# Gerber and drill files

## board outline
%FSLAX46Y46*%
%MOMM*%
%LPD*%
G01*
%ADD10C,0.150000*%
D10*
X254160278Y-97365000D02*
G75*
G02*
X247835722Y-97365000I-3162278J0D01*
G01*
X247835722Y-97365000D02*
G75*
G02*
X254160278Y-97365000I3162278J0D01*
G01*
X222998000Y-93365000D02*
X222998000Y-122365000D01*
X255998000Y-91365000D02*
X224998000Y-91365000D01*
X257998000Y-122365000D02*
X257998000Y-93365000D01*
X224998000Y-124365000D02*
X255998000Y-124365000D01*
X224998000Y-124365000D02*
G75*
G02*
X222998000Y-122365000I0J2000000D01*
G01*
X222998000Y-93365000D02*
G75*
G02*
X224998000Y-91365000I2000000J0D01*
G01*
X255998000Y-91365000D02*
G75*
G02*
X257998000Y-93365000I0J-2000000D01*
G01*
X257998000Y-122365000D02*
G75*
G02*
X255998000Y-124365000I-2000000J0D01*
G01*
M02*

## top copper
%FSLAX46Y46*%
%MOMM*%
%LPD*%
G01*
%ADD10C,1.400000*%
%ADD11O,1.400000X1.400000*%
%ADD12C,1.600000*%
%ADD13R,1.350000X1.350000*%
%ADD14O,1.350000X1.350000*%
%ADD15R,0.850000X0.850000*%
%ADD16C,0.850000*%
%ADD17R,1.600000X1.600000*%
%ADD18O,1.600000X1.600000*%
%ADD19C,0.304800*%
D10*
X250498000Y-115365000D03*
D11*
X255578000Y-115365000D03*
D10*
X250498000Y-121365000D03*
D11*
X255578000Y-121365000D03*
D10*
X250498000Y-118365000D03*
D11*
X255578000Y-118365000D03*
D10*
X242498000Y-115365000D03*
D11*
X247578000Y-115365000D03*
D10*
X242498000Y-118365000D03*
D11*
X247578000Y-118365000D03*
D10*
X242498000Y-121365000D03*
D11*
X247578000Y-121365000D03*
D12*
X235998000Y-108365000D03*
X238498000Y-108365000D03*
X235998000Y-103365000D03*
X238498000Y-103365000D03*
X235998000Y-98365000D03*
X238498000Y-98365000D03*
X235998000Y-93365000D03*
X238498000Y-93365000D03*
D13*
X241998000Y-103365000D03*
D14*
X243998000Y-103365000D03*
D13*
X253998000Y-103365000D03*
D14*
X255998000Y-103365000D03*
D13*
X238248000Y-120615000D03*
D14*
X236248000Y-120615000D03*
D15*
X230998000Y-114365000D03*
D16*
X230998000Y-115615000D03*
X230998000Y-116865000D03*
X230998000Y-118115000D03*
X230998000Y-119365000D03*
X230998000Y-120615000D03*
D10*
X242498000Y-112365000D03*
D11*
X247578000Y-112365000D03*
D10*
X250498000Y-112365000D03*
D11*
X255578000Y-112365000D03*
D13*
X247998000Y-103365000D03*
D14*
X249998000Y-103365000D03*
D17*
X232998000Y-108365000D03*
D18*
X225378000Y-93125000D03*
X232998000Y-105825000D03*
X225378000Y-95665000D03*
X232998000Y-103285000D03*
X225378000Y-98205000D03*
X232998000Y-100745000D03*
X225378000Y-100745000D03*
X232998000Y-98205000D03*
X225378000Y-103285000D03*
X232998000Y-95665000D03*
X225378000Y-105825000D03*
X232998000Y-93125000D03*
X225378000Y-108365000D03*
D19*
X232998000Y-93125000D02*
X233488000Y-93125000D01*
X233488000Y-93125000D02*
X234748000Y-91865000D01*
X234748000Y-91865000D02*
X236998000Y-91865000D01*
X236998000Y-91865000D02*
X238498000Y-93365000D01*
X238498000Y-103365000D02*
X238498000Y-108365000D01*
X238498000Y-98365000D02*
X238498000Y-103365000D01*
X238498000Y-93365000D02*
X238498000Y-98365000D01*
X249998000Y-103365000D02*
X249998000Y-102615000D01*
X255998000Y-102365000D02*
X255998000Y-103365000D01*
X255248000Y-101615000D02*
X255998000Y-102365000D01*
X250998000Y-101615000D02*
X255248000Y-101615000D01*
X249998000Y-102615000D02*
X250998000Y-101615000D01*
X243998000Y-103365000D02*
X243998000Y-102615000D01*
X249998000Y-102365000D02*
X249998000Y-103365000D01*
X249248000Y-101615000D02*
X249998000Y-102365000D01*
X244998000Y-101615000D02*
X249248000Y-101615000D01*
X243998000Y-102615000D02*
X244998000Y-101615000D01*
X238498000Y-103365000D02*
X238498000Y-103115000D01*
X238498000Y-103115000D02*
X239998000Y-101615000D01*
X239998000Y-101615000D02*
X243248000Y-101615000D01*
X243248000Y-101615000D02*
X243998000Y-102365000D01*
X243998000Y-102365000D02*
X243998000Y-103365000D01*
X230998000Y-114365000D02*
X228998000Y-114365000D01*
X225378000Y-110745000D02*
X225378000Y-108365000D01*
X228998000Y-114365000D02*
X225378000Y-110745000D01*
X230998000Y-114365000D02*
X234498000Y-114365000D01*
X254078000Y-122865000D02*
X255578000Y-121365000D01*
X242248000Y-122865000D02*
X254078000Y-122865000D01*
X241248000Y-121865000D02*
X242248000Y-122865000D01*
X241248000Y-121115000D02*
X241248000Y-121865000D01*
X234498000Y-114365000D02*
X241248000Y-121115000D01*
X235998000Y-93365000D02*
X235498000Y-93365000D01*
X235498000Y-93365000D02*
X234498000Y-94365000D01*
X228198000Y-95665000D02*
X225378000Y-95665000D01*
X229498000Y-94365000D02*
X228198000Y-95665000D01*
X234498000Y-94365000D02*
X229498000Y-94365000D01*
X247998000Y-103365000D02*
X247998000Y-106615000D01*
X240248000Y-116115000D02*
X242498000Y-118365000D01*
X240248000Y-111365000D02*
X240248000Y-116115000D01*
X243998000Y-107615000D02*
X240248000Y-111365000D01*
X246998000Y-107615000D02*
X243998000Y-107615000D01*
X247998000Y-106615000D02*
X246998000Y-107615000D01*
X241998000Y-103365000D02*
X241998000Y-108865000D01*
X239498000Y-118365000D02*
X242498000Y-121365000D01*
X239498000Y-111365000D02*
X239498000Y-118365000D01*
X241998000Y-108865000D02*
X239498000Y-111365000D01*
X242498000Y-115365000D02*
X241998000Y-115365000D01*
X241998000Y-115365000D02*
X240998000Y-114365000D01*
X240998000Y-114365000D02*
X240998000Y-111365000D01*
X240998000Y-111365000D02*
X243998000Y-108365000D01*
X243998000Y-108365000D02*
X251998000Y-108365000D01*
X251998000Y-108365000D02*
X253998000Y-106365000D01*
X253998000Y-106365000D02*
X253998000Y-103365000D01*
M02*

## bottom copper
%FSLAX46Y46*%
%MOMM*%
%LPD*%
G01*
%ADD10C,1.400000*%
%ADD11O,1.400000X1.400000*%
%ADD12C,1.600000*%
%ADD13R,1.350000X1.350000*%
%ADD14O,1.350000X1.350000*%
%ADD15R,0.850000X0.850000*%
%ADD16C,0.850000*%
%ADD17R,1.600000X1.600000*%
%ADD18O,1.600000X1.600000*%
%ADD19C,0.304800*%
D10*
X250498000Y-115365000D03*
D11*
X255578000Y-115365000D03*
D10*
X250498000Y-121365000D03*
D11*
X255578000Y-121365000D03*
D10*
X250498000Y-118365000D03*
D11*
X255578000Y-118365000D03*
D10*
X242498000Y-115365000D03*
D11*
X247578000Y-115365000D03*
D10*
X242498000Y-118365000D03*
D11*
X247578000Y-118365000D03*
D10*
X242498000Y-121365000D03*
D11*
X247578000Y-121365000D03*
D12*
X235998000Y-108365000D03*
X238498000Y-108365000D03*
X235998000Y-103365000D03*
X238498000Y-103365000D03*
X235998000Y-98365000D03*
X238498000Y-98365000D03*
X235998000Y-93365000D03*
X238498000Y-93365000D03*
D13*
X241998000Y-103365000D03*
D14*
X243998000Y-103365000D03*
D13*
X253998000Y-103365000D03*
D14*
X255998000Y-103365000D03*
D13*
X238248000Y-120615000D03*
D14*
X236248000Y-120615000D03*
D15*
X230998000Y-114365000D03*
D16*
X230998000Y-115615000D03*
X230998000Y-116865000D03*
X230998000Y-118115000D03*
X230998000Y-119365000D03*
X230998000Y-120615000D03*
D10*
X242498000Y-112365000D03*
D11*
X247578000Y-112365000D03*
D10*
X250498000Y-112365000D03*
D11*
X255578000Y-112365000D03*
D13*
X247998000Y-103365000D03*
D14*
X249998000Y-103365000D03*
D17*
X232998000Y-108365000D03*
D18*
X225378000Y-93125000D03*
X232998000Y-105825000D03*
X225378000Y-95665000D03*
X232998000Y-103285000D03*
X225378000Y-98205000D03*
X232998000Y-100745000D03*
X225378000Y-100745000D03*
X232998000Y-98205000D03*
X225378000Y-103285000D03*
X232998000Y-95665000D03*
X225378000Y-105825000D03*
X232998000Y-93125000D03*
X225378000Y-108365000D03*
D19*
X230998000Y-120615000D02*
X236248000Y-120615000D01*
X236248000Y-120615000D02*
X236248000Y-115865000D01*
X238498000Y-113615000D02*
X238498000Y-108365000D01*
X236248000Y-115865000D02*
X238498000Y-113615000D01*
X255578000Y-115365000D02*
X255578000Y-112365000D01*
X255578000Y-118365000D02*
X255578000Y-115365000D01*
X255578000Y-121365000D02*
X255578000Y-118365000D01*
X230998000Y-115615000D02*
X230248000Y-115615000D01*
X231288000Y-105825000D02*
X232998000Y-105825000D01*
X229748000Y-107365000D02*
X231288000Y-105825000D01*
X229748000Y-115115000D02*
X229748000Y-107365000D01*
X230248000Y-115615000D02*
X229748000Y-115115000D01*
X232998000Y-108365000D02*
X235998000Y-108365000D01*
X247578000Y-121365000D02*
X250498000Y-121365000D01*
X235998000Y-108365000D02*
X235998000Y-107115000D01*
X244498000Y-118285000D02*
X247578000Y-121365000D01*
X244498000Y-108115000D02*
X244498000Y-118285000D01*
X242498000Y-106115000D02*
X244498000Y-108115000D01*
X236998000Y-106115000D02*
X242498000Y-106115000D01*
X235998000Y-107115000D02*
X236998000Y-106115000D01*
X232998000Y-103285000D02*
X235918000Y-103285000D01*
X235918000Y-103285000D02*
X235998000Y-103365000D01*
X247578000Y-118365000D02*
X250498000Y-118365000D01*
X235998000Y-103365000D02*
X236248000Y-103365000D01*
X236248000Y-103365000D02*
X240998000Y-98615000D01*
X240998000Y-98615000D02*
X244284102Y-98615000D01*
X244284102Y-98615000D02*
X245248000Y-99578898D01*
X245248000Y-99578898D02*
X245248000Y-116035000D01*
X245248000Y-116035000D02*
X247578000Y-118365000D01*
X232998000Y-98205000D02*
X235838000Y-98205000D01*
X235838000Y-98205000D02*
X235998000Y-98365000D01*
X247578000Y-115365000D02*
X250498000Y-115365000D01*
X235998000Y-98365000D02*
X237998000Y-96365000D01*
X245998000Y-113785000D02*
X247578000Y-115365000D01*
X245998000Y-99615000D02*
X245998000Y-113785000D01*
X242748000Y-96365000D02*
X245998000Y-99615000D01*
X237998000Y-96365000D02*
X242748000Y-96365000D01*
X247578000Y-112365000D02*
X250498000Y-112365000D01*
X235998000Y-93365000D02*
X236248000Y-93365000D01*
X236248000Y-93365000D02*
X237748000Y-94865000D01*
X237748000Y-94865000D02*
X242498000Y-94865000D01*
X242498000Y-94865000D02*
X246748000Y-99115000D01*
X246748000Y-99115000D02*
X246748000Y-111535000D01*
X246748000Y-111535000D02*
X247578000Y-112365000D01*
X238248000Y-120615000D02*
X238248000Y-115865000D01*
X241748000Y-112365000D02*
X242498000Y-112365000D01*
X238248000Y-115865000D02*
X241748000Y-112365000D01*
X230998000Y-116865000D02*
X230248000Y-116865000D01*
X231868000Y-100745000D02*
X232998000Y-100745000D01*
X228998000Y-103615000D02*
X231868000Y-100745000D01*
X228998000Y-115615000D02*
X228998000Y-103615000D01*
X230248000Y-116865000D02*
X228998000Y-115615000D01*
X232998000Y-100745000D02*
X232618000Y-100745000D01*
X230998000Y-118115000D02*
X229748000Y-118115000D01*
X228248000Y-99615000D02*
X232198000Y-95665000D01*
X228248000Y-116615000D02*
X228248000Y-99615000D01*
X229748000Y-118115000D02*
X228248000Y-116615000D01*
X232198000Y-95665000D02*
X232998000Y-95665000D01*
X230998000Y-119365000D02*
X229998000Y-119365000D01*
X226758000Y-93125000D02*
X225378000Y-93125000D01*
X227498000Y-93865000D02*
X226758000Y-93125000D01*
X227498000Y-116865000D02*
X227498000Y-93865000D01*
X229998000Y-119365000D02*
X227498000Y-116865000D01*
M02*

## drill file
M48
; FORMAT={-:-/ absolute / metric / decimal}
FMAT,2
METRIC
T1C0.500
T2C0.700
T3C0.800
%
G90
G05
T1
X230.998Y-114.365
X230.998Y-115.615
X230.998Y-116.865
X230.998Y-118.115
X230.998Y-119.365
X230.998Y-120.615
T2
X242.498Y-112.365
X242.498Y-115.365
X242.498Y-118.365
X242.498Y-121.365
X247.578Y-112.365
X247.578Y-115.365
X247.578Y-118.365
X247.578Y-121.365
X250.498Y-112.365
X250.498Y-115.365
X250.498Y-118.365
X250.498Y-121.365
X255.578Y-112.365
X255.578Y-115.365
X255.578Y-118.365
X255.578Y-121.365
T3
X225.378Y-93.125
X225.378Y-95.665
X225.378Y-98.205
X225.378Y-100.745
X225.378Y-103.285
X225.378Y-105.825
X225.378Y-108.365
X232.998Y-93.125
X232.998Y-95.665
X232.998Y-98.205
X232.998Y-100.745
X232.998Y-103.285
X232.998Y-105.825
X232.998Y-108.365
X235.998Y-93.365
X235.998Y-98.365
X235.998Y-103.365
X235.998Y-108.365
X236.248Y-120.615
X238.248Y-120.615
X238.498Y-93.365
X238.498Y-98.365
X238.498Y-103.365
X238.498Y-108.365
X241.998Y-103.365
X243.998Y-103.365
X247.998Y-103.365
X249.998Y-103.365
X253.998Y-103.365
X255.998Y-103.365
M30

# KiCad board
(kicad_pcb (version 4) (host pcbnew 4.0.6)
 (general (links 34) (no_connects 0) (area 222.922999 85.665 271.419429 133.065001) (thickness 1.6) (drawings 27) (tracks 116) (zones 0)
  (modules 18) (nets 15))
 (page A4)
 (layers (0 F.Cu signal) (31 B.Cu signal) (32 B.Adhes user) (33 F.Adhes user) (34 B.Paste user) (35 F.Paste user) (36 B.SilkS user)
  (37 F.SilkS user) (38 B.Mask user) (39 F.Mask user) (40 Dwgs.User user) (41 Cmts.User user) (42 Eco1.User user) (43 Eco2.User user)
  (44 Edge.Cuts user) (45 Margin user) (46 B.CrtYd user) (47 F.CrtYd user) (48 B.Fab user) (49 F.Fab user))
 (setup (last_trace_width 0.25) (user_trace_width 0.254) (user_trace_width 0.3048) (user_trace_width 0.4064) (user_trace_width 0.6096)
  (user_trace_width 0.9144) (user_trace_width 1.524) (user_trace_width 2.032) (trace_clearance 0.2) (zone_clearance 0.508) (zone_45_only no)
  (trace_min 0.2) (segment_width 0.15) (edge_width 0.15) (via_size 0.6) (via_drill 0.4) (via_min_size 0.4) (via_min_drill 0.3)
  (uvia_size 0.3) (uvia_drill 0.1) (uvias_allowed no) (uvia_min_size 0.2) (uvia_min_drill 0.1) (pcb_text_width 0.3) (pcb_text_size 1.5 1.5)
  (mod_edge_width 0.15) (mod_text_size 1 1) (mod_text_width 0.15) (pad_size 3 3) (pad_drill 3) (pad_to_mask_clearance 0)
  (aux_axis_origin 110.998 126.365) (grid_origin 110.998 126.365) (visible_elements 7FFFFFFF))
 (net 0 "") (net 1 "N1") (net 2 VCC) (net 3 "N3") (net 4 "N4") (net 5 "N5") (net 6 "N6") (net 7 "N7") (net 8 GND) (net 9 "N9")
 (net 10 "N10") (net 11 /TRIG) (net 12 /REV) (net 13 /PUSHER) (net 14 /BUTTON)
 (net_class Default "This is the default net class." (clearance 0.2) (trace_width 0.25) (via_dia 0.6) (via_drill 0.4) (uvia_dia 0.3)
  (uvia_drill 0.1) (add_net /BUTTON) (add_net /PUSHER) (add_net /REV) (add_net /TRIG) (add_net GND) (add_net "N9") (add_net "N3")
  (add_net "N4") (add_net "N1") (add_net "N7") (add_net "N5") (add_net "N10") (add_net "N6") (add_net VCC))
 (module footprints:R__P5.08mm (layer F.Cu) (at 252.998 115.365)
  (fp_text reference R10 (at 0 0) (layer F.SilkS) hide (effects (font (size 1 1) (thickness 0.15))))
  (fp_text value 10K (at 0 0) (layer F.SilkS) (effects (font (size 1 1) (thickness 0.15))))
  (pad 1 thru_hole circle (at -2.5 0) (size 1.4 1.4) (drill 0.7) (layers *.Cu *.Mask) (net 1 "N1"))
  (pad 2 thru_hole oval (at 2.58 0) (size 1.4 1.4) (drill 0.7) (layers *.Cu *.Mask) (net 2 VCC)))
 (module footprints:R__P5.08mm (layer F.Cu) (at 252.998 121.365)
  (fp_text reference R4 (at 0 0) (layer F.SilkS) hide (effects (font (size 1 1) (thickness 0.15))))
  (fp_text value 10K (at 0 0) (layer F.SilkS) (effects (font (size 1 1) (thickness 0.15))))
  (pad 1 thru_hole circle (at -2.5 0) (size 1.4 1.4) (drill 0.7) (layers *.Cu *.Mask) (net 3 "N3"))
  (pad 2 thru_hole oval (at 2.58 0) (size 1.4 1.4) (drill 0.7) (layers *.Cu *.Mask) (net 2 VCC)))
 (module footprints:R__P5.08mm (layer F.Cu) (at 252.998 118.365)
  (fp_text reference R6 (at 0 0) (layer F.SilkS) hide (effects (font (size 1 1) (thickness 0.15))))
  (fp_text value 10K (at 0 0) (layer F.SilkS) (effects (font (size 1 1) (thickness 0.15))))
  (pad 1 thru_hole circle (at -2.5 0) (size 1.4 1.4) (drill 0.7) (layers *.Cu *.Mask) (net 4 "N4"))
  (pad 2 thru_hole oval (at 2.58 0) (size 1.4 1.4) (drill 0.7) (layers *.Cu *.Mask) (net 2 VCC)))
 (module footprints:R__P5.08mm (layer F.Cu) (at 244.998 115.365)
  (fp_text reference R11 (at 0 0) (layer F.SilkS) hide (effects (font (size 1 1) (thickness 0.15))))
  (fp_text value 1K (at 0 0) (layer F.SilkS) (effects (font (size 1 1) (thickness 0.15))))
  (pad 1 thru_hole circle (at -2.5 0) (size 1.4 1.4) (drill 0.7) (layers *.Cu *.Mask) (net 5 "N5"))
  (pad 2 thru_hole oval (at 2.58 0) (size 1.4 1.4) (drill 0.7) (layers *.Cu *.Mask) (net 1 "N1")))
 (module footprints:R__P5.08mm (layer F.Cu) (at 244.998 118.365)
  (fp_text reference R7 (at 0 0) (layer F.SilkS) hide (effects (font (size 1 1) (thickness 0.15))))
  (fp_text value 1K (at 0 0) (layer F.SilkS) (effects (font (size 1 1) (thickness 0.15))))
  (pad 1 thru_hole circle (at -2.5 0) (size 1.4 1.4) (drill 0.7) (layers *.Cu *.Mask) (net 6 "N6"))
  (pad 2 thru_hole oval (at 2.58 0) (size 1.4 1.4) (drill 0.7) (layers *.Cu *.Mask) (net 4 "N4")))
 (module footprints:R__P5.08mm (layer F.Cu) (at 244.998 121.365)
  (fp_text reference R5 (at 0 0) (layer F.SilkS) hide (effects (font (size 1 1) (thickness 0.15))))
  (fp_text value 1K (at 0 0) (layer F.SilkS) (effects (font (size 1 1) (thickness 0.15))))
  (pad 1 thru_hole circle (at -2.5 0) (size 1.4 1.4) (drill 0.7) (layers *.Cu *.Mask) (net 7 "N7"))
  (pad 2 thru_hole oval (at 2.58 0) (size 1.4 1.4) (drill 0.7) (layers *.Cu *.Mask) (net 3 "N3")))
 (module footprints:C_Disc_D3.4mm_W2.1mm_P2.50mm (layer F.Cu) (at 235.998 108.365)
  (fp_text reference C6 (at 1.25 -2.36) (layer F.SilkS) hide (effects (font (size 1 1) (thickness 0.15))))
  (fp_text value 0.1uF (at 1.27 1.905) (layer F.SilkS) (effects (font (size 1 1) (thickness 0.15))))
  (pad 1 thru_hole circle (at 0 0) (size 1.6 1.6) (drill 0.8) (layers *.Cu *.Mask) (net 3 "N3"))
  (pad 2 thru_hole circle (at 2.5 0) (size 1.6 1.6) (drill 0.8) (layers *.Cu *.Mask) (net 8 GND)))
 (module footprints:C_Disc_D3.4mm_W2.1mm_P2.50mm (layer F.Cu) (at 235.998 103.365)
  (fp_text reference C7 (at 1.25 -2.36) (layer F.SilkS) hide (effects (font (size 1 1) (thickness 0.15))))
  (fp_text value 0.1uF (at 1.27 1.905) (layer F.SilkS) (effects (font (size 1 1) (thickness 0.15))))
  (pad 1 thru_hole circle (at 0 0) (size 1.6 1.6) (drill 0.8) (layers *.Cu *.Mask) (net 4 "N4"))
  (pad 2 thru_hole circle (at 2.5 0) (size 1.6 1.6) (drill 0.8) (layers *.Cu *.Mask) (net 8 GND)))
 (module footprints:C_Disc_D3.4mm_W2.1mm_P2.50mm (layer F.Cu) (at 235.998 98.365)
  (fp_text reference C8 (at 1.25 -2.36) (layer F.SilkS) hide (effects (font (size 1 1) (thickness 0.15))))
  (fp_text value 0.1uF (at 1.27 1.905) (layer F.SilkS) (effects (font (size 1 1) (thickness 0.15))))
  (pad 1 thru_hole circle (at 0 0) (size 1.6 1.6) (drill 0.8) (layers *.Cu *.Mask) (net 1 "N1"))
  (pad 2 thru_hole circle (at 2.5 0) (size 1.6 1.6) (drill 0.8) (layers *.Cu *.Mask) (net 8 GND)))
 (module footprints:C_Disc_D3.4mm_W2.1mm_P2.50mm (layer F.Cu) (at 235.998 93.365)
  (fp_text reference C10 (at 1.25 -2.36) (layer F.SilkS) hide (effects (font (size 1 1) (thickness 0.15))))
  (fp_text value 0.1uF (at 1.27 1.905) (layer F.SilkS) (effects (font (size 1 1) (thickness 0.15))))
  (pad 1 thru_hole circle (at 0 0) (size 1.6 1.6) (drill 0.8) (layers *.Cu *.Mask) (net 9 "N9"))
  (pad 2 thru_hole circle (at 2.5 0) (size 1.6 1.6) (drill 0.8) (layers *.Cu *.Mask) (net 8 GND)))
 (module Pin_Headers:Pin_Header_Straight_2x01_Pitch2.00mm (layer F.Cu) (at 241.998 103.365)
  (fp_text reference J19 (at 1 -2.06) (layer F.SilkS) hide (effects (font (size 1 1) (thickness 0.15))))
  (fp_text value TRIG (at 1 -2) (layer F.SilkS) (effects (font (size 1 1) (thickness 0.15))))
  (pad 1 thru_hole rect (at 0 0) (size 1.35 1.35) (drill 0.8) (layers *.Cu *.Mask) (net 7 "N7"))
  (pad 2 thru_hole oval (at 2 0) (size 1.35 1.35) (drill 0.8) (layers *.Cu *.Mask) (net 8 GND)))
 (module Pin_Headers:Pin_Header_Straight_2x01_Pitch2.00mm (layer F.Cu) (at 253.998 103.365)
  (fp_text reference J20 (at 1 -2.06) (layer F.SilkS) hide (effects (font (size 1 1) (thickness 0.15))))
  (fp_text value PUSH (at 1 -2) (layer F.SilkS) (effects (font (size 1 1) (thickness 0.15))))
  (pad 1 thru_hole rect (at 0 0) (size 1.35 1.35) (drill 0.8) (layers *.Cu *.Mask) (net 5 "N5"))
  (pad 2 thru_hole oval (at 2 0) (size 1.35 1.35) (drill 0.8) (layers *.Cu *.Mask) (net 8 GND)))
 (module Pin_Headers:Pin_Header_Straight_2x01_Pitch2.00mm (layer F.Cu) (at 238.248 120.615 180)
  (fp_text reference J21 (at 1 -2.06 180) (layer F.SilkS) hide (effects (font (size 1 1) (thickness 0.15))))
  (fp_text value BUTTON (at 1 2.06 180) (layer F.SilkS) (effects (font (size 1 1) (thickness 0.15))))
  (pad 1 thru_hole rect (at 0 0 180) (size 1.35 1.35) (drill 0.8) (layers *.Cu *.Mask) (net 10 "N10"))
  (pad 2 thru_hole oval (at 2 0 180) (size 1.35 1.35) (drill 0.8) (layers *.Cu *.Mask) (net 8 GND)))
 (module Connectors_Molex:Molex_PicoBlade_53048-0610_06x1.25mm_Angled (layer F.Cu) (at 230.998 114.365 270)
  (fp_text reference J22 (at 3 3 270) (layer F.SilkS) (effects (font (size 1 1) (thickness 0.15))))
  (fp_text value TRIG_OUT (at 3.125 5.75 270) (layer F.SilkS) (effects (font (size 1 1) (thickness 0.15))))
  (pad 1 thru_hole rect (at 0 0 270) (size 0.85 0.85) (drill 0.5) (layers *.Cu *.Mask) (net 2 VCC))
  (pad 2 thru_hole circle (at 1.25 0 270) (size 0.85 0.85) (drill 0.5) (layers *.Cu *.Mask) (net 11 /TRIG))
  (pad 3 thru_hole circle (at 2.5 0 270) (size 0.85 0.85) (drill 0.5) (layers *.Cu *.Mask) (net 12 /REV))
  (pad 4 thru_hole circle (at 3.75 0 270) (size 0.85 0.85) (drill 0.5) (layers *.Cu *.Mask) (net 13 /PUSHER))
  (pad 5 thru_hole circle (at 5 0 270) (size 0.85 0.85) (drill 0.5) (layers *.Cu *.Mask) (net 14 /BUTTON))
  (pad 6 thru_hole circle (at 6.25 0 270) (size 0.85 0.85) (drill 0.5) (layers *.Cu *.Mask) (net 8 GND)))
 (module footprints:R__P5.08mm (layer F.Cu) (at 244.998 112.365)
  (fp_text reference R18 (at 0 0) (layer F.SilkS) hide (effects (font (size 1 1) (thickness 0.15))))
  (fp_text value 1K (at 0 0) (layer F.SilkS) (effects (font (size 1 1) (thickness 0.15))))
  (pad 1 thru_hole circle (at -2.5 0) (size 1.4 1.4) (drill 0.7) (layers *.Cu *.Mask) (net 10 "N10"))
  (pad 2 thru_hole oval (at 2.58 0) (size 1.4 1.4) (drill 0.7) (layers *.Cu *.Mask) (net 9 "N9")))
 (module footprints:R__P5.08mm (layer F.Cu) (at 252.998 112.365)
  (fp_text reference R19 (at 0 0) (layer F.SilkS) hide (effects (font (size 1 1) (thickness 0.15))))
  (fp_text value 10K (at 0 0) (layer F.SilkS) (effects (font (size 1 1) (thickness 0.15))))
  (pad 1 thru_hole circle (at -2.5 0) (size 1.4 1.4) (drill 0.7) (layers *.Cu *.Mask) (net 9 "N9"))
  (pad 2 thru_hole oval (at 2.58 0) (size 1.4 1.4) (drill 0.7) (layers *.Cu *.Mask) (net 2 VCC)))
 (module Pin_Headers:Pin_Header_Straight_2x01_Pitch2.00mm (layer F.Cu) (at 247.998 103.365)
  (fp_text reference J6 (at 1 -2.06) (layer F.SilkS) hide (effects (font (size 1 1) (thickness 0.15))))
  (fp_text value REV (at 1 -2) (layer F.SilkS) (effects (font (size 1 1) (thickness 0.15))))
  (pad 1 thru_hole rect (at 0 0) (size 1.35 1.35) (drill 0.8) (layers *.Cu *.Mask) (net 6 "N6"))
  (pad 2 thru_hole oval (at 2 0) (size 1.35 1.35) (drill 0.8) (layers *.Cu *.Mask) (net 8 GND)))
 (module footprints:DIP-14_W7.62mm (layer F.Cu) (at 232.998 108.365 180)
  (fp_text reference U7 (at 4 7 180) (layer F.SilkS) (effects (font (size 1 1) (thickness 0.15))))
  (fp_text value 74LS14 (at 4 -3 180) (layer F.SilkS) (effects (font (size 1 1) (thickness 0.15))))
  (pad 1 thru_hole rect (at 0 0 180) (size 1.6 1.6) (drill 0.8) (layers *.Cu *.Mask) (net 3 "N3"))
  (pad 8 thru_hole oval (at 7.62 15.24 180) (size 1.6 1.6) (drill 0.8) (layers *.Cu *.Mask) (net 14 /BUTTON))
  (pad 2 thru_hole oval (at 0 2.54 180) (size 1.6 1.6) (drill 0.8) (layers *.Cu *.Mask) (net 11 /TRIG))
  (pad 9 thru_hole oval (at 7.62 12.7 180) (size 1.6 1.6) (drill 0.8) (layers *.Cu *.Mask) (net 9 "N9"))
  (pad 3 thru_hole oval (at 0 5.08 180) (size 1.6 1.6) (drill 0.8) (layers *.Cu *.Mask) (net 4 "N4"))
  (pad 10 thru_hole oval (at 7.62 10.16 180) (size 1.6 1.6) (drill 0.8) (layers *.Cu *.Mask))
  (pad 4 thru_hole oval (at 0 7.62 180) (size 1.6 1.6) (drill 0.8) (layers *.Cu *.Mask) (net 12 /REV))
  (pad 11 thru_hole oval (at 7.62 7.62 180) (size 1.6 1.6) (drill 0.8) (layers *.Cu *.Mask))
  (pad 5 thru_hole oval (at 0 10.16 180) (size 1.6 1.6) (drill 0.8) (layers *.Cu *.Mask) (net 1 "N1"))
  (pad 12 thru_hole oval (at 7.62 5.08 180) (size 1.6 1.6) (drill 0.8) (layers *.Cu *.Mask))
  (pad 6 thru_hole oval (at 0 12.7 180) (size 1.6 1.6) (drill 0.8) (layers *.Cu *.Mask) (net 13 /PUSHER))
  (pad 13 thru_hole oval (at 7.62 2.54 180) (size 1.6 1.6) (drill 0.8) (layers *.Cu *.Mask))
  (pad 7 thru_hole oval (at 0 15.24 180) (size 1.6 1.6) (drill 0.8) (layers *.Cu *.Mask) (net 8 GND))
  (pad 14 thru_hole oval (at 7.62 0 180) (size 1.6 1.6) (drill 0.8) (layers *.Cu *.Mask) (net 2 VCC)))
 (gr_circle (center 250.998 97.365) (end 251.998 94.365) (layer Edge.Cuts) (width 0.15))
 (gr_line (start 222.998 93.365) (end 222.998 122.365) (angle 90) (layer Edge.Cuts) (width 0.15))
 (gr_line (start 255.998 91.365) (end 224.998 91.365) (angle 90) (layer Edge.Cuts) (width 0.15))
 (gr_line (start 257.998 122.365) (end 257.998 93.365) (angle 90) (layer Edge.Cuts) (width 0.15))
 (gr_line (start 224.998 124.365) (end 255.998 124.365) (angle 90) (layer Edge.Cuts) (width 0.15))
 (gr_arc (start 224.998 122.365) (end 224.998 124.365) (angle 90) (layer Edge.Cuts) (width 0.15))
 (gr_arc (start 224.998 93.365) (end 222.998 93.365) (angle 90) (layer Edge.Cuts) (width 0.15))
 (gr_arc (start 255.998 93.365) (end 255.998 91.365) (angle 90) (layer Edge.Cuts) (width 0.15))
 (gr_arc (start 255.998 122.365) (end 257.998 122.365) (angle 90) (layer Edge.Cuts) (width 0.15))
 (segment (start 232.998 93.125) (end 233.488 93.125) (width 0.3048) (layer F.Cu) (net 8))
 (segment (start 233.488 93.125) (end 234.748 91.865) (width 0.3048) (layer F.Cu) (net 8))
 (segment (start 234.748 91.865) (end 236.998 91.865) (width 0.3048) (layer F.Cu) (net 8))
 (segment (start 236.998 91.865) (end 238.498 93.365) (width 0.3048) (layer F.Cu) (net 8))
 (segment (start 230.998 120.615) (end 236.248 120.615) (width 0.3048) (layer B.Cu) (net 8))
 (segment (start 236.248 120.615) (end 236.248 115.865) (width 0.3048) (layer B.Cu) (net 8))
 (segment (start 238.498 113.615) (end 238.498 108.365) (width 0.3048) (layer B.Cu) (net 8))
 (segment (start 236.248 115.865) (end 238.498 113.615) (width 0.3048) (layer B.Cu) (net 8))
 (segment (start 238.498 103.365) (end 238.498 108.365) (width 0.3048) (layer F.Cu) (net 8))
 (segment (start 238.498 98.365) (end 238.498 103.365) (width 0.3048) (layer F.Cu) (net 8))
 (segment (start 238.498 93.365) (end 238.498 98.365) (width 0.3048) (layer F.Cu) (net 8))
 (segment (start 249.998 103.365) (end 249.998 102.615) (width 0.3048) (layer F.Cu) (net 8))
 (segment (start 255.998 102.365) (end 255.998 103.365) (width 0.3048) (layer F.Cu) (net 8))
 (segment (start 255.248 101.615) (end 255.998 102.365) (width 0.3048) (layer F.Cu) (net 8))
 (segment (start 250.998 101.615) (end 255.248 101.615) (width 0.3048) (layer F.Cu) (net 8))
 (segment (start 249.998 102.615) (end 250.998 101.615) (width 0.3048) (layer F.Cu) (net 8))
 (segment (start 243.998 103.365) (end 243.998 102.615) (width 0.3048) (layer F.Cu) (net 8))
 (segment (start 249.998 102.365) (end 249.998 103.365) (width 0.3048) (layer F.Cu) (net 8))
 (segment (start 249.248 101.615) (end 249.998 102.365) (width 0.3048) (layer F.Cu) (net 8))
 (segment (start 244.998 101.615) (end 249.248 101.615) (width 0.3048) (layer F.Cu) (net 8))
 (segment (start 243.998 102.615) (end 244.998 101.615) (width 0.3048) (layer F.Cu) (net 8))
 (segment (start 238.498 103.365) (end 238.498 103.115) (width 0.3048) (layer F.Cu) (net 8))
 (segment (start 238.498 103.115) (end 239.998 101.615) (width 0.3048) (layer F.Cu) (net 8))
 (segment (start 239.998 101.615) (end 243.248 101.615) (width 0.3048) (layer F.Cu) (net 8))
 (segment (start 243.248 101.615) (end 243.998 102.365) (width 0.3048) (layer F.Cu) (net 8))
 (segment (start 243.998 102.365) (end 243.998 103.365) (width 0.3048) (layer F.Cu) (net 8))
 (segment (start 230.998 114.365) (end 228.998 114.365) (width 0.3048) (layer F.Cu) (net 2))
 (segment (start 225.378 110.745) (end 225.378 108.365) (width 0.3048) (layer F.Cu) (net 2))
 (segment (start 228.998 114.365) (end 225.378 110.745) (width 0.3048) (layer F.Cu) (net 2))
 (segment (start 230.998 114.365) (end 234.498 114.365) (width 0.3048) (layer F.Cu) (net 2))
 (segment (start 254.078 122.865) (end 255.578 121.365) (width 0.3048) (layer F.Cu) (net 2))
 (segment (start 242.248 122.865) (end 254.078 122.865) (width 0.3048) (layer F.Cu) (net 2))
 (segment (start 241.248 121.865) (end 242.248 122.865) (width 0.3048) (layer F.Cu) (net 2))
 (segment (start 241.248 121.115) (end 241.248 121.865) (width 0.3048) (layer F.Cu) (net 2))
 (segment (start 234.498 114.365) (end 241.248 121.115) (width 0.3048) (layer F.Cu) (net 2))
 (segment (start 255.578 115.365) (end 255.578 112.365) (width 0.3048) (layer B.Cu) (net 2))
 (segment (start 255.578 118.365) (end 255.578 115.365) (width 0.3048) (layer B.Cu) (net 2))
 (segment (start 255.578 121.365) (end 255.578 118.365) (width 0.3048) (layer B.Cu) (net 2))
 (segment (start 230.998 115.615) (end 230.248 115.615) (width 0.3048) (layer B.Cu) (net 11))
 (segment (start 231.288 105.825) (end 232.998 105.825) (width 0.3048) (layer B.Cu) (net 11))
 (segment (start 229.748 107.365) (end 231.288 105.825) (width 0.3048) (layer B.Cu) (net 11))
 (segment (start 229.748 115.115) (end 229.748 107.365) (width 0.3048) (layer B.Cu) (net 11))
 (segment (start 230.248 115.615) (end 229.748 115.115) (width 0.3048) (layer B.Cu) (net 11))
 (segment (start 232.998 108.365) (end 235.998 108.365) (width 0.3048) (layer B.Cu) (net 3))
 (segment (start 247.578 121.365) (end 250.498 121.365) (width 0.3048) (layer B.Cu) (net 3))
 (segment (start 235.998 108.365) (end 235.998 107.115) (width 0.3048) (layer B.Cu) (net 3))
 (segment (start 244.498 118.285) (end 247.578 121.365) (width 0.3048) (layer B.Cu) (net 3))
 (segment (start 244.498 108.115) (end 244.498 118.285) (width 0.3048) (layer B.Cu) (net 3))
 (segment (start 242.498 106.115) (end 244.498 108.115) (width 0.3048) (layer B.Cu) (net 3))
 (segment (start 236.998 106.115) (end 242.498 106.115) (width 0.3048) (layer B.Cu) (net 3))
 (segment (start 235.998 107.115) (end 236.998 106.115) (width 0.3048) (layer B.Cu) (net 3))
 (segment (start 232.998 103.285) (end 235.918 103.285) (width 0.3048) (layer B.Cu) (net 4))
 (segment (start 235.918 103.285) (end 235.998 103.365) (width 0.3048) (layer B.Cu) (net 4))
 (segment (start 247.578 118.365) (end 250.498 118.365) (width 0.3048) (layer B.Cu) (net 4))
 (segment (start 235.998 103.365) (end 236.248 103.365) (width 0.3048) (layer B.Cu) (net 4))
 (segment (start 236.248 103.365) (end 240.998 98.615) (width 0.3048) (layer B.Cu) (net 4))
 (segment (start 240.998 98.615) (end 244.284102 98.615) (width 0.3048) (layer B.Cu) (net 4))
 (segment (start 244.284102 98.615) (end 245.248 99.578898) (width 0.3048) (layer B.Cu) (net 4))
 (segment (start 245.248 99.578898) (end 245.248 116.035) (width 0.3048) (layer B.Cu) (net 4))
 (segment (start 245.248 116.035) (end 247.578 118.365) (width 0.3048) (layer B.Cu) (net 4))
 (segment (start 232.998 98.205) (end 235.838 98.205) (width 0.3048) (layer B.Cu) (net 1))
 (segment (start 235.838 98.205) (end 235.998 98.365) (width 0.3048) (layer B.Cu) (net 1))
 (segment (start 247.578 115.365) (end 250.498 115.365) (width 0.3048) (layer B.Cu) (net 1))
 (segment (start 235.998 98.365) (end 237.998 96.365) (width 0.3048) (layer B.Cu) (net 1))
 (segment (start 245.998 113.785) (end 247.578 115.365) (width 0.3048) (layer B.Cu) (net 1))
 (segment (start 245.998 99.615) (end 245.998 113.785) (width 0.3048) (layer B.Cu) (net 1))
 (segment (start 242.748 96.365) (end 245.998 99.615) (width 0.3048) (layer B.Cu) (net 1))
 (segment (start 237.998 96.365) (end 242.748 96.365) (width 0.3048) (layer B.Cu) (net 1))
 (segment (start 235.998 93.365) (end 235.498 93.365) (width 0.3048) (layer F.Cu) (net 9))
 (segment (start 235.498 93.365) (end 234.498 94.365) (width 0.3048) (layer F.Cu) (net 9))
 (segment (start 228.198 95.665) (end 225.378 95.665) (width 0.3048) (layer F.Cu) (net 9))
 (segment (start 229.498 94.365) (end 228.198 95.665) (width 0.3048) (layer F.Cu) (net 9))
 (segment (start 234.498 94.365) (end 229.498 94.365) (width 0.3048) (layer F.Cu) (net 9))
 (segment (start 247.578 112.365) (end 250.498 112.365) (width 0.3048) (layer B.Cu) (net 9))
 (segment (start 235.998 93.365) (end 236.248 93.365) (width 0.3048) (layer B.Cu) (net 9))
 (segment (start 236.248 93.365) (end 237.748 94.865) (width 0.3048) (layer B.Cu) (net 9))
 (segment (start 237.748 94.865) (end 242.498 94.865) (width 0.3048) (layer B.Cu) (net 9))
 (segment (start 242.498 94.865) (end 246.748 99.115) (width 0.3048) (layer B.Cu) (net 9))
 (segment (start 246.748 99.115) (end 246.748 111.535) (width 0.3048) (layer B.Cu) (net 9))
 (segment (start 246.748 111.535) (end 247.578 112.365) (width 0.3048) (layer B.Cu) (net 9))
 (segment (start 247.998 103.365) (end 247.998 106.615) (width 0.3048) (layer F.Cu) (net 6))
 (segment (start 240.248 116.115) (end 242.498 118.365) (width 0.3048) (layer F.Cu) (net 6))
 (segment (start 240.248 111.365) (end 240.248 116.115) (width 0.3048) (layer F.Cu) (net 6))
 (segment (start 243.998 107.615) (end 240.248 111.365) (width 0.3048) (layer F.Cu) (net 6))
 (segment (start 246.998 107.615) (end 243.998 107.615) (width 0.3048) (layer F.Cu) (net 6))
 (segment (start 247.998 106.615) (end 246.998 107.615) (width 0.3048) (layer F.Cu) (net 6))
 (segment (start 241.998 103.365) (end 241.998 108.865) (width 0.3048) (layer F.Cu) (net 7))
 (segment (start 239.498 118.365) (end 242.498 121.365) (width 0.3048) (layer F.Cu) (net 7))
 (segment (start 239.498 111.365) (end 239.498 118.365) (width 0.3048) (layer F.Cu) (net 7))
 (segment (start 241.998 108.865) (end 239.498 111.365) (width 0.3048) (layer F.Cu) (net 7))
 (segment (start 242.498 115.365) (end 241.998 115.365) (width 0.3048) (layer F.Cu) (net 5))
 (segment (start 241.998 115.365) (end 240.998 114.365) (width 0.3048) (layer F.Cu) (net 5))
 (segment (start 240.998 114.365) (end 240.998 111.365) (width 0.3048) (layer F.Cu) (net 5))
 (segment (start 240.998 111.365) (end 243.998 108.365) (width 0.3048) (layer F.Cu) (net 5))
 (segment (start 243.998 108.365) (end 251.998 108.365) (width 0.3048) (layer F.Cu) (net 5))
 (segment (start 251.998 108.365) (end 253.998 106.365) (width 0.3048) (layer F.Cu) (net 5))
 (segment (start 253.998 106.365) (end 253.998 103.365) (width 0.3048) (layer F.Cu) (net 5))
 (segment (start 238.248 120.615) (end 238.248 115.865) (width 0.3048) (layer B.Cu) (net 10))
 (segment (start 241.748 112.365) (end 242.498 112.365) (width 0.3048) (layer B.Cu) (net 10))
 (segment (start 238.248 115.865) (end 241.748 112.365) (width 0.3048) (layer B.Cu) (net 10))
 (segment (start 230.998 116.865) (end 230.248 116.865) (width 0.3048) (layer B.Cu) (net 12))
 (segment (start 231.868 100.745) (end 232.998 100.745) (width 0.3048) (layer B.Cu) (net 12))
 (segment (start 228.998 103.615) (end 231.868 100.745) (width 0.3048) (layer B.Cu) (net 12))
 (segment (start 228.998 115.615) (end 228.998 103.615) (width 0.3048) (layer B.Cu) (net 12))
 (segment (start 230.248 116.865) (end 228.998 115.615) (width 0.3048) (layer B.Cu) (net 12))
 (segment (start 232.998 100.745) (end 232.618 100.745) (width 0.3048) (layer B.Cu) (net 12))
 (segment (start 230.998 118.115) (end 229.748 118.115) (width 0.3048) (layer B.Cu) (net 13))
 (segment (start 228.248 99.615) (end 232.198 95.665) (width 0.3048) (layer B.Cu) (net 13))
 (segment (start 228.248 116.615) (end 228.248 99.615) (width 0.3048) (layer B.Cu) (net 13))
 (segment (start 229.748 118.115) (end 228.248 116.615) (width 0.3048) (layer B.Cu) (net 13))
 (segment (start 232.198 95.665) (end 232.998 95.665) (width 0.3048) (layer B.Cu) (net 13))
 (segment (start 230.998 119.365) (end 229.998 119.365) (width 0.3048) (layer B.Cu) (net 14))
 (segment (start 226.758 93.125) (end 225.378 93.125) (width 0.3048) (layer B.Cu) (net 14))
 (segment (start 227.498 93.865) (end 226.758 93.125) (width 0.3048) (layer B.Cu) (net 14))
 (segment (start 227.498 116.865) (end 227.498 93.865) (width 0.3048) (layer B.Cu) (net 14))
 (segment (start 229.998 119.365) (end 227.498 116.865) (width 0.3048) (layer B.Cu) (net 14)))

